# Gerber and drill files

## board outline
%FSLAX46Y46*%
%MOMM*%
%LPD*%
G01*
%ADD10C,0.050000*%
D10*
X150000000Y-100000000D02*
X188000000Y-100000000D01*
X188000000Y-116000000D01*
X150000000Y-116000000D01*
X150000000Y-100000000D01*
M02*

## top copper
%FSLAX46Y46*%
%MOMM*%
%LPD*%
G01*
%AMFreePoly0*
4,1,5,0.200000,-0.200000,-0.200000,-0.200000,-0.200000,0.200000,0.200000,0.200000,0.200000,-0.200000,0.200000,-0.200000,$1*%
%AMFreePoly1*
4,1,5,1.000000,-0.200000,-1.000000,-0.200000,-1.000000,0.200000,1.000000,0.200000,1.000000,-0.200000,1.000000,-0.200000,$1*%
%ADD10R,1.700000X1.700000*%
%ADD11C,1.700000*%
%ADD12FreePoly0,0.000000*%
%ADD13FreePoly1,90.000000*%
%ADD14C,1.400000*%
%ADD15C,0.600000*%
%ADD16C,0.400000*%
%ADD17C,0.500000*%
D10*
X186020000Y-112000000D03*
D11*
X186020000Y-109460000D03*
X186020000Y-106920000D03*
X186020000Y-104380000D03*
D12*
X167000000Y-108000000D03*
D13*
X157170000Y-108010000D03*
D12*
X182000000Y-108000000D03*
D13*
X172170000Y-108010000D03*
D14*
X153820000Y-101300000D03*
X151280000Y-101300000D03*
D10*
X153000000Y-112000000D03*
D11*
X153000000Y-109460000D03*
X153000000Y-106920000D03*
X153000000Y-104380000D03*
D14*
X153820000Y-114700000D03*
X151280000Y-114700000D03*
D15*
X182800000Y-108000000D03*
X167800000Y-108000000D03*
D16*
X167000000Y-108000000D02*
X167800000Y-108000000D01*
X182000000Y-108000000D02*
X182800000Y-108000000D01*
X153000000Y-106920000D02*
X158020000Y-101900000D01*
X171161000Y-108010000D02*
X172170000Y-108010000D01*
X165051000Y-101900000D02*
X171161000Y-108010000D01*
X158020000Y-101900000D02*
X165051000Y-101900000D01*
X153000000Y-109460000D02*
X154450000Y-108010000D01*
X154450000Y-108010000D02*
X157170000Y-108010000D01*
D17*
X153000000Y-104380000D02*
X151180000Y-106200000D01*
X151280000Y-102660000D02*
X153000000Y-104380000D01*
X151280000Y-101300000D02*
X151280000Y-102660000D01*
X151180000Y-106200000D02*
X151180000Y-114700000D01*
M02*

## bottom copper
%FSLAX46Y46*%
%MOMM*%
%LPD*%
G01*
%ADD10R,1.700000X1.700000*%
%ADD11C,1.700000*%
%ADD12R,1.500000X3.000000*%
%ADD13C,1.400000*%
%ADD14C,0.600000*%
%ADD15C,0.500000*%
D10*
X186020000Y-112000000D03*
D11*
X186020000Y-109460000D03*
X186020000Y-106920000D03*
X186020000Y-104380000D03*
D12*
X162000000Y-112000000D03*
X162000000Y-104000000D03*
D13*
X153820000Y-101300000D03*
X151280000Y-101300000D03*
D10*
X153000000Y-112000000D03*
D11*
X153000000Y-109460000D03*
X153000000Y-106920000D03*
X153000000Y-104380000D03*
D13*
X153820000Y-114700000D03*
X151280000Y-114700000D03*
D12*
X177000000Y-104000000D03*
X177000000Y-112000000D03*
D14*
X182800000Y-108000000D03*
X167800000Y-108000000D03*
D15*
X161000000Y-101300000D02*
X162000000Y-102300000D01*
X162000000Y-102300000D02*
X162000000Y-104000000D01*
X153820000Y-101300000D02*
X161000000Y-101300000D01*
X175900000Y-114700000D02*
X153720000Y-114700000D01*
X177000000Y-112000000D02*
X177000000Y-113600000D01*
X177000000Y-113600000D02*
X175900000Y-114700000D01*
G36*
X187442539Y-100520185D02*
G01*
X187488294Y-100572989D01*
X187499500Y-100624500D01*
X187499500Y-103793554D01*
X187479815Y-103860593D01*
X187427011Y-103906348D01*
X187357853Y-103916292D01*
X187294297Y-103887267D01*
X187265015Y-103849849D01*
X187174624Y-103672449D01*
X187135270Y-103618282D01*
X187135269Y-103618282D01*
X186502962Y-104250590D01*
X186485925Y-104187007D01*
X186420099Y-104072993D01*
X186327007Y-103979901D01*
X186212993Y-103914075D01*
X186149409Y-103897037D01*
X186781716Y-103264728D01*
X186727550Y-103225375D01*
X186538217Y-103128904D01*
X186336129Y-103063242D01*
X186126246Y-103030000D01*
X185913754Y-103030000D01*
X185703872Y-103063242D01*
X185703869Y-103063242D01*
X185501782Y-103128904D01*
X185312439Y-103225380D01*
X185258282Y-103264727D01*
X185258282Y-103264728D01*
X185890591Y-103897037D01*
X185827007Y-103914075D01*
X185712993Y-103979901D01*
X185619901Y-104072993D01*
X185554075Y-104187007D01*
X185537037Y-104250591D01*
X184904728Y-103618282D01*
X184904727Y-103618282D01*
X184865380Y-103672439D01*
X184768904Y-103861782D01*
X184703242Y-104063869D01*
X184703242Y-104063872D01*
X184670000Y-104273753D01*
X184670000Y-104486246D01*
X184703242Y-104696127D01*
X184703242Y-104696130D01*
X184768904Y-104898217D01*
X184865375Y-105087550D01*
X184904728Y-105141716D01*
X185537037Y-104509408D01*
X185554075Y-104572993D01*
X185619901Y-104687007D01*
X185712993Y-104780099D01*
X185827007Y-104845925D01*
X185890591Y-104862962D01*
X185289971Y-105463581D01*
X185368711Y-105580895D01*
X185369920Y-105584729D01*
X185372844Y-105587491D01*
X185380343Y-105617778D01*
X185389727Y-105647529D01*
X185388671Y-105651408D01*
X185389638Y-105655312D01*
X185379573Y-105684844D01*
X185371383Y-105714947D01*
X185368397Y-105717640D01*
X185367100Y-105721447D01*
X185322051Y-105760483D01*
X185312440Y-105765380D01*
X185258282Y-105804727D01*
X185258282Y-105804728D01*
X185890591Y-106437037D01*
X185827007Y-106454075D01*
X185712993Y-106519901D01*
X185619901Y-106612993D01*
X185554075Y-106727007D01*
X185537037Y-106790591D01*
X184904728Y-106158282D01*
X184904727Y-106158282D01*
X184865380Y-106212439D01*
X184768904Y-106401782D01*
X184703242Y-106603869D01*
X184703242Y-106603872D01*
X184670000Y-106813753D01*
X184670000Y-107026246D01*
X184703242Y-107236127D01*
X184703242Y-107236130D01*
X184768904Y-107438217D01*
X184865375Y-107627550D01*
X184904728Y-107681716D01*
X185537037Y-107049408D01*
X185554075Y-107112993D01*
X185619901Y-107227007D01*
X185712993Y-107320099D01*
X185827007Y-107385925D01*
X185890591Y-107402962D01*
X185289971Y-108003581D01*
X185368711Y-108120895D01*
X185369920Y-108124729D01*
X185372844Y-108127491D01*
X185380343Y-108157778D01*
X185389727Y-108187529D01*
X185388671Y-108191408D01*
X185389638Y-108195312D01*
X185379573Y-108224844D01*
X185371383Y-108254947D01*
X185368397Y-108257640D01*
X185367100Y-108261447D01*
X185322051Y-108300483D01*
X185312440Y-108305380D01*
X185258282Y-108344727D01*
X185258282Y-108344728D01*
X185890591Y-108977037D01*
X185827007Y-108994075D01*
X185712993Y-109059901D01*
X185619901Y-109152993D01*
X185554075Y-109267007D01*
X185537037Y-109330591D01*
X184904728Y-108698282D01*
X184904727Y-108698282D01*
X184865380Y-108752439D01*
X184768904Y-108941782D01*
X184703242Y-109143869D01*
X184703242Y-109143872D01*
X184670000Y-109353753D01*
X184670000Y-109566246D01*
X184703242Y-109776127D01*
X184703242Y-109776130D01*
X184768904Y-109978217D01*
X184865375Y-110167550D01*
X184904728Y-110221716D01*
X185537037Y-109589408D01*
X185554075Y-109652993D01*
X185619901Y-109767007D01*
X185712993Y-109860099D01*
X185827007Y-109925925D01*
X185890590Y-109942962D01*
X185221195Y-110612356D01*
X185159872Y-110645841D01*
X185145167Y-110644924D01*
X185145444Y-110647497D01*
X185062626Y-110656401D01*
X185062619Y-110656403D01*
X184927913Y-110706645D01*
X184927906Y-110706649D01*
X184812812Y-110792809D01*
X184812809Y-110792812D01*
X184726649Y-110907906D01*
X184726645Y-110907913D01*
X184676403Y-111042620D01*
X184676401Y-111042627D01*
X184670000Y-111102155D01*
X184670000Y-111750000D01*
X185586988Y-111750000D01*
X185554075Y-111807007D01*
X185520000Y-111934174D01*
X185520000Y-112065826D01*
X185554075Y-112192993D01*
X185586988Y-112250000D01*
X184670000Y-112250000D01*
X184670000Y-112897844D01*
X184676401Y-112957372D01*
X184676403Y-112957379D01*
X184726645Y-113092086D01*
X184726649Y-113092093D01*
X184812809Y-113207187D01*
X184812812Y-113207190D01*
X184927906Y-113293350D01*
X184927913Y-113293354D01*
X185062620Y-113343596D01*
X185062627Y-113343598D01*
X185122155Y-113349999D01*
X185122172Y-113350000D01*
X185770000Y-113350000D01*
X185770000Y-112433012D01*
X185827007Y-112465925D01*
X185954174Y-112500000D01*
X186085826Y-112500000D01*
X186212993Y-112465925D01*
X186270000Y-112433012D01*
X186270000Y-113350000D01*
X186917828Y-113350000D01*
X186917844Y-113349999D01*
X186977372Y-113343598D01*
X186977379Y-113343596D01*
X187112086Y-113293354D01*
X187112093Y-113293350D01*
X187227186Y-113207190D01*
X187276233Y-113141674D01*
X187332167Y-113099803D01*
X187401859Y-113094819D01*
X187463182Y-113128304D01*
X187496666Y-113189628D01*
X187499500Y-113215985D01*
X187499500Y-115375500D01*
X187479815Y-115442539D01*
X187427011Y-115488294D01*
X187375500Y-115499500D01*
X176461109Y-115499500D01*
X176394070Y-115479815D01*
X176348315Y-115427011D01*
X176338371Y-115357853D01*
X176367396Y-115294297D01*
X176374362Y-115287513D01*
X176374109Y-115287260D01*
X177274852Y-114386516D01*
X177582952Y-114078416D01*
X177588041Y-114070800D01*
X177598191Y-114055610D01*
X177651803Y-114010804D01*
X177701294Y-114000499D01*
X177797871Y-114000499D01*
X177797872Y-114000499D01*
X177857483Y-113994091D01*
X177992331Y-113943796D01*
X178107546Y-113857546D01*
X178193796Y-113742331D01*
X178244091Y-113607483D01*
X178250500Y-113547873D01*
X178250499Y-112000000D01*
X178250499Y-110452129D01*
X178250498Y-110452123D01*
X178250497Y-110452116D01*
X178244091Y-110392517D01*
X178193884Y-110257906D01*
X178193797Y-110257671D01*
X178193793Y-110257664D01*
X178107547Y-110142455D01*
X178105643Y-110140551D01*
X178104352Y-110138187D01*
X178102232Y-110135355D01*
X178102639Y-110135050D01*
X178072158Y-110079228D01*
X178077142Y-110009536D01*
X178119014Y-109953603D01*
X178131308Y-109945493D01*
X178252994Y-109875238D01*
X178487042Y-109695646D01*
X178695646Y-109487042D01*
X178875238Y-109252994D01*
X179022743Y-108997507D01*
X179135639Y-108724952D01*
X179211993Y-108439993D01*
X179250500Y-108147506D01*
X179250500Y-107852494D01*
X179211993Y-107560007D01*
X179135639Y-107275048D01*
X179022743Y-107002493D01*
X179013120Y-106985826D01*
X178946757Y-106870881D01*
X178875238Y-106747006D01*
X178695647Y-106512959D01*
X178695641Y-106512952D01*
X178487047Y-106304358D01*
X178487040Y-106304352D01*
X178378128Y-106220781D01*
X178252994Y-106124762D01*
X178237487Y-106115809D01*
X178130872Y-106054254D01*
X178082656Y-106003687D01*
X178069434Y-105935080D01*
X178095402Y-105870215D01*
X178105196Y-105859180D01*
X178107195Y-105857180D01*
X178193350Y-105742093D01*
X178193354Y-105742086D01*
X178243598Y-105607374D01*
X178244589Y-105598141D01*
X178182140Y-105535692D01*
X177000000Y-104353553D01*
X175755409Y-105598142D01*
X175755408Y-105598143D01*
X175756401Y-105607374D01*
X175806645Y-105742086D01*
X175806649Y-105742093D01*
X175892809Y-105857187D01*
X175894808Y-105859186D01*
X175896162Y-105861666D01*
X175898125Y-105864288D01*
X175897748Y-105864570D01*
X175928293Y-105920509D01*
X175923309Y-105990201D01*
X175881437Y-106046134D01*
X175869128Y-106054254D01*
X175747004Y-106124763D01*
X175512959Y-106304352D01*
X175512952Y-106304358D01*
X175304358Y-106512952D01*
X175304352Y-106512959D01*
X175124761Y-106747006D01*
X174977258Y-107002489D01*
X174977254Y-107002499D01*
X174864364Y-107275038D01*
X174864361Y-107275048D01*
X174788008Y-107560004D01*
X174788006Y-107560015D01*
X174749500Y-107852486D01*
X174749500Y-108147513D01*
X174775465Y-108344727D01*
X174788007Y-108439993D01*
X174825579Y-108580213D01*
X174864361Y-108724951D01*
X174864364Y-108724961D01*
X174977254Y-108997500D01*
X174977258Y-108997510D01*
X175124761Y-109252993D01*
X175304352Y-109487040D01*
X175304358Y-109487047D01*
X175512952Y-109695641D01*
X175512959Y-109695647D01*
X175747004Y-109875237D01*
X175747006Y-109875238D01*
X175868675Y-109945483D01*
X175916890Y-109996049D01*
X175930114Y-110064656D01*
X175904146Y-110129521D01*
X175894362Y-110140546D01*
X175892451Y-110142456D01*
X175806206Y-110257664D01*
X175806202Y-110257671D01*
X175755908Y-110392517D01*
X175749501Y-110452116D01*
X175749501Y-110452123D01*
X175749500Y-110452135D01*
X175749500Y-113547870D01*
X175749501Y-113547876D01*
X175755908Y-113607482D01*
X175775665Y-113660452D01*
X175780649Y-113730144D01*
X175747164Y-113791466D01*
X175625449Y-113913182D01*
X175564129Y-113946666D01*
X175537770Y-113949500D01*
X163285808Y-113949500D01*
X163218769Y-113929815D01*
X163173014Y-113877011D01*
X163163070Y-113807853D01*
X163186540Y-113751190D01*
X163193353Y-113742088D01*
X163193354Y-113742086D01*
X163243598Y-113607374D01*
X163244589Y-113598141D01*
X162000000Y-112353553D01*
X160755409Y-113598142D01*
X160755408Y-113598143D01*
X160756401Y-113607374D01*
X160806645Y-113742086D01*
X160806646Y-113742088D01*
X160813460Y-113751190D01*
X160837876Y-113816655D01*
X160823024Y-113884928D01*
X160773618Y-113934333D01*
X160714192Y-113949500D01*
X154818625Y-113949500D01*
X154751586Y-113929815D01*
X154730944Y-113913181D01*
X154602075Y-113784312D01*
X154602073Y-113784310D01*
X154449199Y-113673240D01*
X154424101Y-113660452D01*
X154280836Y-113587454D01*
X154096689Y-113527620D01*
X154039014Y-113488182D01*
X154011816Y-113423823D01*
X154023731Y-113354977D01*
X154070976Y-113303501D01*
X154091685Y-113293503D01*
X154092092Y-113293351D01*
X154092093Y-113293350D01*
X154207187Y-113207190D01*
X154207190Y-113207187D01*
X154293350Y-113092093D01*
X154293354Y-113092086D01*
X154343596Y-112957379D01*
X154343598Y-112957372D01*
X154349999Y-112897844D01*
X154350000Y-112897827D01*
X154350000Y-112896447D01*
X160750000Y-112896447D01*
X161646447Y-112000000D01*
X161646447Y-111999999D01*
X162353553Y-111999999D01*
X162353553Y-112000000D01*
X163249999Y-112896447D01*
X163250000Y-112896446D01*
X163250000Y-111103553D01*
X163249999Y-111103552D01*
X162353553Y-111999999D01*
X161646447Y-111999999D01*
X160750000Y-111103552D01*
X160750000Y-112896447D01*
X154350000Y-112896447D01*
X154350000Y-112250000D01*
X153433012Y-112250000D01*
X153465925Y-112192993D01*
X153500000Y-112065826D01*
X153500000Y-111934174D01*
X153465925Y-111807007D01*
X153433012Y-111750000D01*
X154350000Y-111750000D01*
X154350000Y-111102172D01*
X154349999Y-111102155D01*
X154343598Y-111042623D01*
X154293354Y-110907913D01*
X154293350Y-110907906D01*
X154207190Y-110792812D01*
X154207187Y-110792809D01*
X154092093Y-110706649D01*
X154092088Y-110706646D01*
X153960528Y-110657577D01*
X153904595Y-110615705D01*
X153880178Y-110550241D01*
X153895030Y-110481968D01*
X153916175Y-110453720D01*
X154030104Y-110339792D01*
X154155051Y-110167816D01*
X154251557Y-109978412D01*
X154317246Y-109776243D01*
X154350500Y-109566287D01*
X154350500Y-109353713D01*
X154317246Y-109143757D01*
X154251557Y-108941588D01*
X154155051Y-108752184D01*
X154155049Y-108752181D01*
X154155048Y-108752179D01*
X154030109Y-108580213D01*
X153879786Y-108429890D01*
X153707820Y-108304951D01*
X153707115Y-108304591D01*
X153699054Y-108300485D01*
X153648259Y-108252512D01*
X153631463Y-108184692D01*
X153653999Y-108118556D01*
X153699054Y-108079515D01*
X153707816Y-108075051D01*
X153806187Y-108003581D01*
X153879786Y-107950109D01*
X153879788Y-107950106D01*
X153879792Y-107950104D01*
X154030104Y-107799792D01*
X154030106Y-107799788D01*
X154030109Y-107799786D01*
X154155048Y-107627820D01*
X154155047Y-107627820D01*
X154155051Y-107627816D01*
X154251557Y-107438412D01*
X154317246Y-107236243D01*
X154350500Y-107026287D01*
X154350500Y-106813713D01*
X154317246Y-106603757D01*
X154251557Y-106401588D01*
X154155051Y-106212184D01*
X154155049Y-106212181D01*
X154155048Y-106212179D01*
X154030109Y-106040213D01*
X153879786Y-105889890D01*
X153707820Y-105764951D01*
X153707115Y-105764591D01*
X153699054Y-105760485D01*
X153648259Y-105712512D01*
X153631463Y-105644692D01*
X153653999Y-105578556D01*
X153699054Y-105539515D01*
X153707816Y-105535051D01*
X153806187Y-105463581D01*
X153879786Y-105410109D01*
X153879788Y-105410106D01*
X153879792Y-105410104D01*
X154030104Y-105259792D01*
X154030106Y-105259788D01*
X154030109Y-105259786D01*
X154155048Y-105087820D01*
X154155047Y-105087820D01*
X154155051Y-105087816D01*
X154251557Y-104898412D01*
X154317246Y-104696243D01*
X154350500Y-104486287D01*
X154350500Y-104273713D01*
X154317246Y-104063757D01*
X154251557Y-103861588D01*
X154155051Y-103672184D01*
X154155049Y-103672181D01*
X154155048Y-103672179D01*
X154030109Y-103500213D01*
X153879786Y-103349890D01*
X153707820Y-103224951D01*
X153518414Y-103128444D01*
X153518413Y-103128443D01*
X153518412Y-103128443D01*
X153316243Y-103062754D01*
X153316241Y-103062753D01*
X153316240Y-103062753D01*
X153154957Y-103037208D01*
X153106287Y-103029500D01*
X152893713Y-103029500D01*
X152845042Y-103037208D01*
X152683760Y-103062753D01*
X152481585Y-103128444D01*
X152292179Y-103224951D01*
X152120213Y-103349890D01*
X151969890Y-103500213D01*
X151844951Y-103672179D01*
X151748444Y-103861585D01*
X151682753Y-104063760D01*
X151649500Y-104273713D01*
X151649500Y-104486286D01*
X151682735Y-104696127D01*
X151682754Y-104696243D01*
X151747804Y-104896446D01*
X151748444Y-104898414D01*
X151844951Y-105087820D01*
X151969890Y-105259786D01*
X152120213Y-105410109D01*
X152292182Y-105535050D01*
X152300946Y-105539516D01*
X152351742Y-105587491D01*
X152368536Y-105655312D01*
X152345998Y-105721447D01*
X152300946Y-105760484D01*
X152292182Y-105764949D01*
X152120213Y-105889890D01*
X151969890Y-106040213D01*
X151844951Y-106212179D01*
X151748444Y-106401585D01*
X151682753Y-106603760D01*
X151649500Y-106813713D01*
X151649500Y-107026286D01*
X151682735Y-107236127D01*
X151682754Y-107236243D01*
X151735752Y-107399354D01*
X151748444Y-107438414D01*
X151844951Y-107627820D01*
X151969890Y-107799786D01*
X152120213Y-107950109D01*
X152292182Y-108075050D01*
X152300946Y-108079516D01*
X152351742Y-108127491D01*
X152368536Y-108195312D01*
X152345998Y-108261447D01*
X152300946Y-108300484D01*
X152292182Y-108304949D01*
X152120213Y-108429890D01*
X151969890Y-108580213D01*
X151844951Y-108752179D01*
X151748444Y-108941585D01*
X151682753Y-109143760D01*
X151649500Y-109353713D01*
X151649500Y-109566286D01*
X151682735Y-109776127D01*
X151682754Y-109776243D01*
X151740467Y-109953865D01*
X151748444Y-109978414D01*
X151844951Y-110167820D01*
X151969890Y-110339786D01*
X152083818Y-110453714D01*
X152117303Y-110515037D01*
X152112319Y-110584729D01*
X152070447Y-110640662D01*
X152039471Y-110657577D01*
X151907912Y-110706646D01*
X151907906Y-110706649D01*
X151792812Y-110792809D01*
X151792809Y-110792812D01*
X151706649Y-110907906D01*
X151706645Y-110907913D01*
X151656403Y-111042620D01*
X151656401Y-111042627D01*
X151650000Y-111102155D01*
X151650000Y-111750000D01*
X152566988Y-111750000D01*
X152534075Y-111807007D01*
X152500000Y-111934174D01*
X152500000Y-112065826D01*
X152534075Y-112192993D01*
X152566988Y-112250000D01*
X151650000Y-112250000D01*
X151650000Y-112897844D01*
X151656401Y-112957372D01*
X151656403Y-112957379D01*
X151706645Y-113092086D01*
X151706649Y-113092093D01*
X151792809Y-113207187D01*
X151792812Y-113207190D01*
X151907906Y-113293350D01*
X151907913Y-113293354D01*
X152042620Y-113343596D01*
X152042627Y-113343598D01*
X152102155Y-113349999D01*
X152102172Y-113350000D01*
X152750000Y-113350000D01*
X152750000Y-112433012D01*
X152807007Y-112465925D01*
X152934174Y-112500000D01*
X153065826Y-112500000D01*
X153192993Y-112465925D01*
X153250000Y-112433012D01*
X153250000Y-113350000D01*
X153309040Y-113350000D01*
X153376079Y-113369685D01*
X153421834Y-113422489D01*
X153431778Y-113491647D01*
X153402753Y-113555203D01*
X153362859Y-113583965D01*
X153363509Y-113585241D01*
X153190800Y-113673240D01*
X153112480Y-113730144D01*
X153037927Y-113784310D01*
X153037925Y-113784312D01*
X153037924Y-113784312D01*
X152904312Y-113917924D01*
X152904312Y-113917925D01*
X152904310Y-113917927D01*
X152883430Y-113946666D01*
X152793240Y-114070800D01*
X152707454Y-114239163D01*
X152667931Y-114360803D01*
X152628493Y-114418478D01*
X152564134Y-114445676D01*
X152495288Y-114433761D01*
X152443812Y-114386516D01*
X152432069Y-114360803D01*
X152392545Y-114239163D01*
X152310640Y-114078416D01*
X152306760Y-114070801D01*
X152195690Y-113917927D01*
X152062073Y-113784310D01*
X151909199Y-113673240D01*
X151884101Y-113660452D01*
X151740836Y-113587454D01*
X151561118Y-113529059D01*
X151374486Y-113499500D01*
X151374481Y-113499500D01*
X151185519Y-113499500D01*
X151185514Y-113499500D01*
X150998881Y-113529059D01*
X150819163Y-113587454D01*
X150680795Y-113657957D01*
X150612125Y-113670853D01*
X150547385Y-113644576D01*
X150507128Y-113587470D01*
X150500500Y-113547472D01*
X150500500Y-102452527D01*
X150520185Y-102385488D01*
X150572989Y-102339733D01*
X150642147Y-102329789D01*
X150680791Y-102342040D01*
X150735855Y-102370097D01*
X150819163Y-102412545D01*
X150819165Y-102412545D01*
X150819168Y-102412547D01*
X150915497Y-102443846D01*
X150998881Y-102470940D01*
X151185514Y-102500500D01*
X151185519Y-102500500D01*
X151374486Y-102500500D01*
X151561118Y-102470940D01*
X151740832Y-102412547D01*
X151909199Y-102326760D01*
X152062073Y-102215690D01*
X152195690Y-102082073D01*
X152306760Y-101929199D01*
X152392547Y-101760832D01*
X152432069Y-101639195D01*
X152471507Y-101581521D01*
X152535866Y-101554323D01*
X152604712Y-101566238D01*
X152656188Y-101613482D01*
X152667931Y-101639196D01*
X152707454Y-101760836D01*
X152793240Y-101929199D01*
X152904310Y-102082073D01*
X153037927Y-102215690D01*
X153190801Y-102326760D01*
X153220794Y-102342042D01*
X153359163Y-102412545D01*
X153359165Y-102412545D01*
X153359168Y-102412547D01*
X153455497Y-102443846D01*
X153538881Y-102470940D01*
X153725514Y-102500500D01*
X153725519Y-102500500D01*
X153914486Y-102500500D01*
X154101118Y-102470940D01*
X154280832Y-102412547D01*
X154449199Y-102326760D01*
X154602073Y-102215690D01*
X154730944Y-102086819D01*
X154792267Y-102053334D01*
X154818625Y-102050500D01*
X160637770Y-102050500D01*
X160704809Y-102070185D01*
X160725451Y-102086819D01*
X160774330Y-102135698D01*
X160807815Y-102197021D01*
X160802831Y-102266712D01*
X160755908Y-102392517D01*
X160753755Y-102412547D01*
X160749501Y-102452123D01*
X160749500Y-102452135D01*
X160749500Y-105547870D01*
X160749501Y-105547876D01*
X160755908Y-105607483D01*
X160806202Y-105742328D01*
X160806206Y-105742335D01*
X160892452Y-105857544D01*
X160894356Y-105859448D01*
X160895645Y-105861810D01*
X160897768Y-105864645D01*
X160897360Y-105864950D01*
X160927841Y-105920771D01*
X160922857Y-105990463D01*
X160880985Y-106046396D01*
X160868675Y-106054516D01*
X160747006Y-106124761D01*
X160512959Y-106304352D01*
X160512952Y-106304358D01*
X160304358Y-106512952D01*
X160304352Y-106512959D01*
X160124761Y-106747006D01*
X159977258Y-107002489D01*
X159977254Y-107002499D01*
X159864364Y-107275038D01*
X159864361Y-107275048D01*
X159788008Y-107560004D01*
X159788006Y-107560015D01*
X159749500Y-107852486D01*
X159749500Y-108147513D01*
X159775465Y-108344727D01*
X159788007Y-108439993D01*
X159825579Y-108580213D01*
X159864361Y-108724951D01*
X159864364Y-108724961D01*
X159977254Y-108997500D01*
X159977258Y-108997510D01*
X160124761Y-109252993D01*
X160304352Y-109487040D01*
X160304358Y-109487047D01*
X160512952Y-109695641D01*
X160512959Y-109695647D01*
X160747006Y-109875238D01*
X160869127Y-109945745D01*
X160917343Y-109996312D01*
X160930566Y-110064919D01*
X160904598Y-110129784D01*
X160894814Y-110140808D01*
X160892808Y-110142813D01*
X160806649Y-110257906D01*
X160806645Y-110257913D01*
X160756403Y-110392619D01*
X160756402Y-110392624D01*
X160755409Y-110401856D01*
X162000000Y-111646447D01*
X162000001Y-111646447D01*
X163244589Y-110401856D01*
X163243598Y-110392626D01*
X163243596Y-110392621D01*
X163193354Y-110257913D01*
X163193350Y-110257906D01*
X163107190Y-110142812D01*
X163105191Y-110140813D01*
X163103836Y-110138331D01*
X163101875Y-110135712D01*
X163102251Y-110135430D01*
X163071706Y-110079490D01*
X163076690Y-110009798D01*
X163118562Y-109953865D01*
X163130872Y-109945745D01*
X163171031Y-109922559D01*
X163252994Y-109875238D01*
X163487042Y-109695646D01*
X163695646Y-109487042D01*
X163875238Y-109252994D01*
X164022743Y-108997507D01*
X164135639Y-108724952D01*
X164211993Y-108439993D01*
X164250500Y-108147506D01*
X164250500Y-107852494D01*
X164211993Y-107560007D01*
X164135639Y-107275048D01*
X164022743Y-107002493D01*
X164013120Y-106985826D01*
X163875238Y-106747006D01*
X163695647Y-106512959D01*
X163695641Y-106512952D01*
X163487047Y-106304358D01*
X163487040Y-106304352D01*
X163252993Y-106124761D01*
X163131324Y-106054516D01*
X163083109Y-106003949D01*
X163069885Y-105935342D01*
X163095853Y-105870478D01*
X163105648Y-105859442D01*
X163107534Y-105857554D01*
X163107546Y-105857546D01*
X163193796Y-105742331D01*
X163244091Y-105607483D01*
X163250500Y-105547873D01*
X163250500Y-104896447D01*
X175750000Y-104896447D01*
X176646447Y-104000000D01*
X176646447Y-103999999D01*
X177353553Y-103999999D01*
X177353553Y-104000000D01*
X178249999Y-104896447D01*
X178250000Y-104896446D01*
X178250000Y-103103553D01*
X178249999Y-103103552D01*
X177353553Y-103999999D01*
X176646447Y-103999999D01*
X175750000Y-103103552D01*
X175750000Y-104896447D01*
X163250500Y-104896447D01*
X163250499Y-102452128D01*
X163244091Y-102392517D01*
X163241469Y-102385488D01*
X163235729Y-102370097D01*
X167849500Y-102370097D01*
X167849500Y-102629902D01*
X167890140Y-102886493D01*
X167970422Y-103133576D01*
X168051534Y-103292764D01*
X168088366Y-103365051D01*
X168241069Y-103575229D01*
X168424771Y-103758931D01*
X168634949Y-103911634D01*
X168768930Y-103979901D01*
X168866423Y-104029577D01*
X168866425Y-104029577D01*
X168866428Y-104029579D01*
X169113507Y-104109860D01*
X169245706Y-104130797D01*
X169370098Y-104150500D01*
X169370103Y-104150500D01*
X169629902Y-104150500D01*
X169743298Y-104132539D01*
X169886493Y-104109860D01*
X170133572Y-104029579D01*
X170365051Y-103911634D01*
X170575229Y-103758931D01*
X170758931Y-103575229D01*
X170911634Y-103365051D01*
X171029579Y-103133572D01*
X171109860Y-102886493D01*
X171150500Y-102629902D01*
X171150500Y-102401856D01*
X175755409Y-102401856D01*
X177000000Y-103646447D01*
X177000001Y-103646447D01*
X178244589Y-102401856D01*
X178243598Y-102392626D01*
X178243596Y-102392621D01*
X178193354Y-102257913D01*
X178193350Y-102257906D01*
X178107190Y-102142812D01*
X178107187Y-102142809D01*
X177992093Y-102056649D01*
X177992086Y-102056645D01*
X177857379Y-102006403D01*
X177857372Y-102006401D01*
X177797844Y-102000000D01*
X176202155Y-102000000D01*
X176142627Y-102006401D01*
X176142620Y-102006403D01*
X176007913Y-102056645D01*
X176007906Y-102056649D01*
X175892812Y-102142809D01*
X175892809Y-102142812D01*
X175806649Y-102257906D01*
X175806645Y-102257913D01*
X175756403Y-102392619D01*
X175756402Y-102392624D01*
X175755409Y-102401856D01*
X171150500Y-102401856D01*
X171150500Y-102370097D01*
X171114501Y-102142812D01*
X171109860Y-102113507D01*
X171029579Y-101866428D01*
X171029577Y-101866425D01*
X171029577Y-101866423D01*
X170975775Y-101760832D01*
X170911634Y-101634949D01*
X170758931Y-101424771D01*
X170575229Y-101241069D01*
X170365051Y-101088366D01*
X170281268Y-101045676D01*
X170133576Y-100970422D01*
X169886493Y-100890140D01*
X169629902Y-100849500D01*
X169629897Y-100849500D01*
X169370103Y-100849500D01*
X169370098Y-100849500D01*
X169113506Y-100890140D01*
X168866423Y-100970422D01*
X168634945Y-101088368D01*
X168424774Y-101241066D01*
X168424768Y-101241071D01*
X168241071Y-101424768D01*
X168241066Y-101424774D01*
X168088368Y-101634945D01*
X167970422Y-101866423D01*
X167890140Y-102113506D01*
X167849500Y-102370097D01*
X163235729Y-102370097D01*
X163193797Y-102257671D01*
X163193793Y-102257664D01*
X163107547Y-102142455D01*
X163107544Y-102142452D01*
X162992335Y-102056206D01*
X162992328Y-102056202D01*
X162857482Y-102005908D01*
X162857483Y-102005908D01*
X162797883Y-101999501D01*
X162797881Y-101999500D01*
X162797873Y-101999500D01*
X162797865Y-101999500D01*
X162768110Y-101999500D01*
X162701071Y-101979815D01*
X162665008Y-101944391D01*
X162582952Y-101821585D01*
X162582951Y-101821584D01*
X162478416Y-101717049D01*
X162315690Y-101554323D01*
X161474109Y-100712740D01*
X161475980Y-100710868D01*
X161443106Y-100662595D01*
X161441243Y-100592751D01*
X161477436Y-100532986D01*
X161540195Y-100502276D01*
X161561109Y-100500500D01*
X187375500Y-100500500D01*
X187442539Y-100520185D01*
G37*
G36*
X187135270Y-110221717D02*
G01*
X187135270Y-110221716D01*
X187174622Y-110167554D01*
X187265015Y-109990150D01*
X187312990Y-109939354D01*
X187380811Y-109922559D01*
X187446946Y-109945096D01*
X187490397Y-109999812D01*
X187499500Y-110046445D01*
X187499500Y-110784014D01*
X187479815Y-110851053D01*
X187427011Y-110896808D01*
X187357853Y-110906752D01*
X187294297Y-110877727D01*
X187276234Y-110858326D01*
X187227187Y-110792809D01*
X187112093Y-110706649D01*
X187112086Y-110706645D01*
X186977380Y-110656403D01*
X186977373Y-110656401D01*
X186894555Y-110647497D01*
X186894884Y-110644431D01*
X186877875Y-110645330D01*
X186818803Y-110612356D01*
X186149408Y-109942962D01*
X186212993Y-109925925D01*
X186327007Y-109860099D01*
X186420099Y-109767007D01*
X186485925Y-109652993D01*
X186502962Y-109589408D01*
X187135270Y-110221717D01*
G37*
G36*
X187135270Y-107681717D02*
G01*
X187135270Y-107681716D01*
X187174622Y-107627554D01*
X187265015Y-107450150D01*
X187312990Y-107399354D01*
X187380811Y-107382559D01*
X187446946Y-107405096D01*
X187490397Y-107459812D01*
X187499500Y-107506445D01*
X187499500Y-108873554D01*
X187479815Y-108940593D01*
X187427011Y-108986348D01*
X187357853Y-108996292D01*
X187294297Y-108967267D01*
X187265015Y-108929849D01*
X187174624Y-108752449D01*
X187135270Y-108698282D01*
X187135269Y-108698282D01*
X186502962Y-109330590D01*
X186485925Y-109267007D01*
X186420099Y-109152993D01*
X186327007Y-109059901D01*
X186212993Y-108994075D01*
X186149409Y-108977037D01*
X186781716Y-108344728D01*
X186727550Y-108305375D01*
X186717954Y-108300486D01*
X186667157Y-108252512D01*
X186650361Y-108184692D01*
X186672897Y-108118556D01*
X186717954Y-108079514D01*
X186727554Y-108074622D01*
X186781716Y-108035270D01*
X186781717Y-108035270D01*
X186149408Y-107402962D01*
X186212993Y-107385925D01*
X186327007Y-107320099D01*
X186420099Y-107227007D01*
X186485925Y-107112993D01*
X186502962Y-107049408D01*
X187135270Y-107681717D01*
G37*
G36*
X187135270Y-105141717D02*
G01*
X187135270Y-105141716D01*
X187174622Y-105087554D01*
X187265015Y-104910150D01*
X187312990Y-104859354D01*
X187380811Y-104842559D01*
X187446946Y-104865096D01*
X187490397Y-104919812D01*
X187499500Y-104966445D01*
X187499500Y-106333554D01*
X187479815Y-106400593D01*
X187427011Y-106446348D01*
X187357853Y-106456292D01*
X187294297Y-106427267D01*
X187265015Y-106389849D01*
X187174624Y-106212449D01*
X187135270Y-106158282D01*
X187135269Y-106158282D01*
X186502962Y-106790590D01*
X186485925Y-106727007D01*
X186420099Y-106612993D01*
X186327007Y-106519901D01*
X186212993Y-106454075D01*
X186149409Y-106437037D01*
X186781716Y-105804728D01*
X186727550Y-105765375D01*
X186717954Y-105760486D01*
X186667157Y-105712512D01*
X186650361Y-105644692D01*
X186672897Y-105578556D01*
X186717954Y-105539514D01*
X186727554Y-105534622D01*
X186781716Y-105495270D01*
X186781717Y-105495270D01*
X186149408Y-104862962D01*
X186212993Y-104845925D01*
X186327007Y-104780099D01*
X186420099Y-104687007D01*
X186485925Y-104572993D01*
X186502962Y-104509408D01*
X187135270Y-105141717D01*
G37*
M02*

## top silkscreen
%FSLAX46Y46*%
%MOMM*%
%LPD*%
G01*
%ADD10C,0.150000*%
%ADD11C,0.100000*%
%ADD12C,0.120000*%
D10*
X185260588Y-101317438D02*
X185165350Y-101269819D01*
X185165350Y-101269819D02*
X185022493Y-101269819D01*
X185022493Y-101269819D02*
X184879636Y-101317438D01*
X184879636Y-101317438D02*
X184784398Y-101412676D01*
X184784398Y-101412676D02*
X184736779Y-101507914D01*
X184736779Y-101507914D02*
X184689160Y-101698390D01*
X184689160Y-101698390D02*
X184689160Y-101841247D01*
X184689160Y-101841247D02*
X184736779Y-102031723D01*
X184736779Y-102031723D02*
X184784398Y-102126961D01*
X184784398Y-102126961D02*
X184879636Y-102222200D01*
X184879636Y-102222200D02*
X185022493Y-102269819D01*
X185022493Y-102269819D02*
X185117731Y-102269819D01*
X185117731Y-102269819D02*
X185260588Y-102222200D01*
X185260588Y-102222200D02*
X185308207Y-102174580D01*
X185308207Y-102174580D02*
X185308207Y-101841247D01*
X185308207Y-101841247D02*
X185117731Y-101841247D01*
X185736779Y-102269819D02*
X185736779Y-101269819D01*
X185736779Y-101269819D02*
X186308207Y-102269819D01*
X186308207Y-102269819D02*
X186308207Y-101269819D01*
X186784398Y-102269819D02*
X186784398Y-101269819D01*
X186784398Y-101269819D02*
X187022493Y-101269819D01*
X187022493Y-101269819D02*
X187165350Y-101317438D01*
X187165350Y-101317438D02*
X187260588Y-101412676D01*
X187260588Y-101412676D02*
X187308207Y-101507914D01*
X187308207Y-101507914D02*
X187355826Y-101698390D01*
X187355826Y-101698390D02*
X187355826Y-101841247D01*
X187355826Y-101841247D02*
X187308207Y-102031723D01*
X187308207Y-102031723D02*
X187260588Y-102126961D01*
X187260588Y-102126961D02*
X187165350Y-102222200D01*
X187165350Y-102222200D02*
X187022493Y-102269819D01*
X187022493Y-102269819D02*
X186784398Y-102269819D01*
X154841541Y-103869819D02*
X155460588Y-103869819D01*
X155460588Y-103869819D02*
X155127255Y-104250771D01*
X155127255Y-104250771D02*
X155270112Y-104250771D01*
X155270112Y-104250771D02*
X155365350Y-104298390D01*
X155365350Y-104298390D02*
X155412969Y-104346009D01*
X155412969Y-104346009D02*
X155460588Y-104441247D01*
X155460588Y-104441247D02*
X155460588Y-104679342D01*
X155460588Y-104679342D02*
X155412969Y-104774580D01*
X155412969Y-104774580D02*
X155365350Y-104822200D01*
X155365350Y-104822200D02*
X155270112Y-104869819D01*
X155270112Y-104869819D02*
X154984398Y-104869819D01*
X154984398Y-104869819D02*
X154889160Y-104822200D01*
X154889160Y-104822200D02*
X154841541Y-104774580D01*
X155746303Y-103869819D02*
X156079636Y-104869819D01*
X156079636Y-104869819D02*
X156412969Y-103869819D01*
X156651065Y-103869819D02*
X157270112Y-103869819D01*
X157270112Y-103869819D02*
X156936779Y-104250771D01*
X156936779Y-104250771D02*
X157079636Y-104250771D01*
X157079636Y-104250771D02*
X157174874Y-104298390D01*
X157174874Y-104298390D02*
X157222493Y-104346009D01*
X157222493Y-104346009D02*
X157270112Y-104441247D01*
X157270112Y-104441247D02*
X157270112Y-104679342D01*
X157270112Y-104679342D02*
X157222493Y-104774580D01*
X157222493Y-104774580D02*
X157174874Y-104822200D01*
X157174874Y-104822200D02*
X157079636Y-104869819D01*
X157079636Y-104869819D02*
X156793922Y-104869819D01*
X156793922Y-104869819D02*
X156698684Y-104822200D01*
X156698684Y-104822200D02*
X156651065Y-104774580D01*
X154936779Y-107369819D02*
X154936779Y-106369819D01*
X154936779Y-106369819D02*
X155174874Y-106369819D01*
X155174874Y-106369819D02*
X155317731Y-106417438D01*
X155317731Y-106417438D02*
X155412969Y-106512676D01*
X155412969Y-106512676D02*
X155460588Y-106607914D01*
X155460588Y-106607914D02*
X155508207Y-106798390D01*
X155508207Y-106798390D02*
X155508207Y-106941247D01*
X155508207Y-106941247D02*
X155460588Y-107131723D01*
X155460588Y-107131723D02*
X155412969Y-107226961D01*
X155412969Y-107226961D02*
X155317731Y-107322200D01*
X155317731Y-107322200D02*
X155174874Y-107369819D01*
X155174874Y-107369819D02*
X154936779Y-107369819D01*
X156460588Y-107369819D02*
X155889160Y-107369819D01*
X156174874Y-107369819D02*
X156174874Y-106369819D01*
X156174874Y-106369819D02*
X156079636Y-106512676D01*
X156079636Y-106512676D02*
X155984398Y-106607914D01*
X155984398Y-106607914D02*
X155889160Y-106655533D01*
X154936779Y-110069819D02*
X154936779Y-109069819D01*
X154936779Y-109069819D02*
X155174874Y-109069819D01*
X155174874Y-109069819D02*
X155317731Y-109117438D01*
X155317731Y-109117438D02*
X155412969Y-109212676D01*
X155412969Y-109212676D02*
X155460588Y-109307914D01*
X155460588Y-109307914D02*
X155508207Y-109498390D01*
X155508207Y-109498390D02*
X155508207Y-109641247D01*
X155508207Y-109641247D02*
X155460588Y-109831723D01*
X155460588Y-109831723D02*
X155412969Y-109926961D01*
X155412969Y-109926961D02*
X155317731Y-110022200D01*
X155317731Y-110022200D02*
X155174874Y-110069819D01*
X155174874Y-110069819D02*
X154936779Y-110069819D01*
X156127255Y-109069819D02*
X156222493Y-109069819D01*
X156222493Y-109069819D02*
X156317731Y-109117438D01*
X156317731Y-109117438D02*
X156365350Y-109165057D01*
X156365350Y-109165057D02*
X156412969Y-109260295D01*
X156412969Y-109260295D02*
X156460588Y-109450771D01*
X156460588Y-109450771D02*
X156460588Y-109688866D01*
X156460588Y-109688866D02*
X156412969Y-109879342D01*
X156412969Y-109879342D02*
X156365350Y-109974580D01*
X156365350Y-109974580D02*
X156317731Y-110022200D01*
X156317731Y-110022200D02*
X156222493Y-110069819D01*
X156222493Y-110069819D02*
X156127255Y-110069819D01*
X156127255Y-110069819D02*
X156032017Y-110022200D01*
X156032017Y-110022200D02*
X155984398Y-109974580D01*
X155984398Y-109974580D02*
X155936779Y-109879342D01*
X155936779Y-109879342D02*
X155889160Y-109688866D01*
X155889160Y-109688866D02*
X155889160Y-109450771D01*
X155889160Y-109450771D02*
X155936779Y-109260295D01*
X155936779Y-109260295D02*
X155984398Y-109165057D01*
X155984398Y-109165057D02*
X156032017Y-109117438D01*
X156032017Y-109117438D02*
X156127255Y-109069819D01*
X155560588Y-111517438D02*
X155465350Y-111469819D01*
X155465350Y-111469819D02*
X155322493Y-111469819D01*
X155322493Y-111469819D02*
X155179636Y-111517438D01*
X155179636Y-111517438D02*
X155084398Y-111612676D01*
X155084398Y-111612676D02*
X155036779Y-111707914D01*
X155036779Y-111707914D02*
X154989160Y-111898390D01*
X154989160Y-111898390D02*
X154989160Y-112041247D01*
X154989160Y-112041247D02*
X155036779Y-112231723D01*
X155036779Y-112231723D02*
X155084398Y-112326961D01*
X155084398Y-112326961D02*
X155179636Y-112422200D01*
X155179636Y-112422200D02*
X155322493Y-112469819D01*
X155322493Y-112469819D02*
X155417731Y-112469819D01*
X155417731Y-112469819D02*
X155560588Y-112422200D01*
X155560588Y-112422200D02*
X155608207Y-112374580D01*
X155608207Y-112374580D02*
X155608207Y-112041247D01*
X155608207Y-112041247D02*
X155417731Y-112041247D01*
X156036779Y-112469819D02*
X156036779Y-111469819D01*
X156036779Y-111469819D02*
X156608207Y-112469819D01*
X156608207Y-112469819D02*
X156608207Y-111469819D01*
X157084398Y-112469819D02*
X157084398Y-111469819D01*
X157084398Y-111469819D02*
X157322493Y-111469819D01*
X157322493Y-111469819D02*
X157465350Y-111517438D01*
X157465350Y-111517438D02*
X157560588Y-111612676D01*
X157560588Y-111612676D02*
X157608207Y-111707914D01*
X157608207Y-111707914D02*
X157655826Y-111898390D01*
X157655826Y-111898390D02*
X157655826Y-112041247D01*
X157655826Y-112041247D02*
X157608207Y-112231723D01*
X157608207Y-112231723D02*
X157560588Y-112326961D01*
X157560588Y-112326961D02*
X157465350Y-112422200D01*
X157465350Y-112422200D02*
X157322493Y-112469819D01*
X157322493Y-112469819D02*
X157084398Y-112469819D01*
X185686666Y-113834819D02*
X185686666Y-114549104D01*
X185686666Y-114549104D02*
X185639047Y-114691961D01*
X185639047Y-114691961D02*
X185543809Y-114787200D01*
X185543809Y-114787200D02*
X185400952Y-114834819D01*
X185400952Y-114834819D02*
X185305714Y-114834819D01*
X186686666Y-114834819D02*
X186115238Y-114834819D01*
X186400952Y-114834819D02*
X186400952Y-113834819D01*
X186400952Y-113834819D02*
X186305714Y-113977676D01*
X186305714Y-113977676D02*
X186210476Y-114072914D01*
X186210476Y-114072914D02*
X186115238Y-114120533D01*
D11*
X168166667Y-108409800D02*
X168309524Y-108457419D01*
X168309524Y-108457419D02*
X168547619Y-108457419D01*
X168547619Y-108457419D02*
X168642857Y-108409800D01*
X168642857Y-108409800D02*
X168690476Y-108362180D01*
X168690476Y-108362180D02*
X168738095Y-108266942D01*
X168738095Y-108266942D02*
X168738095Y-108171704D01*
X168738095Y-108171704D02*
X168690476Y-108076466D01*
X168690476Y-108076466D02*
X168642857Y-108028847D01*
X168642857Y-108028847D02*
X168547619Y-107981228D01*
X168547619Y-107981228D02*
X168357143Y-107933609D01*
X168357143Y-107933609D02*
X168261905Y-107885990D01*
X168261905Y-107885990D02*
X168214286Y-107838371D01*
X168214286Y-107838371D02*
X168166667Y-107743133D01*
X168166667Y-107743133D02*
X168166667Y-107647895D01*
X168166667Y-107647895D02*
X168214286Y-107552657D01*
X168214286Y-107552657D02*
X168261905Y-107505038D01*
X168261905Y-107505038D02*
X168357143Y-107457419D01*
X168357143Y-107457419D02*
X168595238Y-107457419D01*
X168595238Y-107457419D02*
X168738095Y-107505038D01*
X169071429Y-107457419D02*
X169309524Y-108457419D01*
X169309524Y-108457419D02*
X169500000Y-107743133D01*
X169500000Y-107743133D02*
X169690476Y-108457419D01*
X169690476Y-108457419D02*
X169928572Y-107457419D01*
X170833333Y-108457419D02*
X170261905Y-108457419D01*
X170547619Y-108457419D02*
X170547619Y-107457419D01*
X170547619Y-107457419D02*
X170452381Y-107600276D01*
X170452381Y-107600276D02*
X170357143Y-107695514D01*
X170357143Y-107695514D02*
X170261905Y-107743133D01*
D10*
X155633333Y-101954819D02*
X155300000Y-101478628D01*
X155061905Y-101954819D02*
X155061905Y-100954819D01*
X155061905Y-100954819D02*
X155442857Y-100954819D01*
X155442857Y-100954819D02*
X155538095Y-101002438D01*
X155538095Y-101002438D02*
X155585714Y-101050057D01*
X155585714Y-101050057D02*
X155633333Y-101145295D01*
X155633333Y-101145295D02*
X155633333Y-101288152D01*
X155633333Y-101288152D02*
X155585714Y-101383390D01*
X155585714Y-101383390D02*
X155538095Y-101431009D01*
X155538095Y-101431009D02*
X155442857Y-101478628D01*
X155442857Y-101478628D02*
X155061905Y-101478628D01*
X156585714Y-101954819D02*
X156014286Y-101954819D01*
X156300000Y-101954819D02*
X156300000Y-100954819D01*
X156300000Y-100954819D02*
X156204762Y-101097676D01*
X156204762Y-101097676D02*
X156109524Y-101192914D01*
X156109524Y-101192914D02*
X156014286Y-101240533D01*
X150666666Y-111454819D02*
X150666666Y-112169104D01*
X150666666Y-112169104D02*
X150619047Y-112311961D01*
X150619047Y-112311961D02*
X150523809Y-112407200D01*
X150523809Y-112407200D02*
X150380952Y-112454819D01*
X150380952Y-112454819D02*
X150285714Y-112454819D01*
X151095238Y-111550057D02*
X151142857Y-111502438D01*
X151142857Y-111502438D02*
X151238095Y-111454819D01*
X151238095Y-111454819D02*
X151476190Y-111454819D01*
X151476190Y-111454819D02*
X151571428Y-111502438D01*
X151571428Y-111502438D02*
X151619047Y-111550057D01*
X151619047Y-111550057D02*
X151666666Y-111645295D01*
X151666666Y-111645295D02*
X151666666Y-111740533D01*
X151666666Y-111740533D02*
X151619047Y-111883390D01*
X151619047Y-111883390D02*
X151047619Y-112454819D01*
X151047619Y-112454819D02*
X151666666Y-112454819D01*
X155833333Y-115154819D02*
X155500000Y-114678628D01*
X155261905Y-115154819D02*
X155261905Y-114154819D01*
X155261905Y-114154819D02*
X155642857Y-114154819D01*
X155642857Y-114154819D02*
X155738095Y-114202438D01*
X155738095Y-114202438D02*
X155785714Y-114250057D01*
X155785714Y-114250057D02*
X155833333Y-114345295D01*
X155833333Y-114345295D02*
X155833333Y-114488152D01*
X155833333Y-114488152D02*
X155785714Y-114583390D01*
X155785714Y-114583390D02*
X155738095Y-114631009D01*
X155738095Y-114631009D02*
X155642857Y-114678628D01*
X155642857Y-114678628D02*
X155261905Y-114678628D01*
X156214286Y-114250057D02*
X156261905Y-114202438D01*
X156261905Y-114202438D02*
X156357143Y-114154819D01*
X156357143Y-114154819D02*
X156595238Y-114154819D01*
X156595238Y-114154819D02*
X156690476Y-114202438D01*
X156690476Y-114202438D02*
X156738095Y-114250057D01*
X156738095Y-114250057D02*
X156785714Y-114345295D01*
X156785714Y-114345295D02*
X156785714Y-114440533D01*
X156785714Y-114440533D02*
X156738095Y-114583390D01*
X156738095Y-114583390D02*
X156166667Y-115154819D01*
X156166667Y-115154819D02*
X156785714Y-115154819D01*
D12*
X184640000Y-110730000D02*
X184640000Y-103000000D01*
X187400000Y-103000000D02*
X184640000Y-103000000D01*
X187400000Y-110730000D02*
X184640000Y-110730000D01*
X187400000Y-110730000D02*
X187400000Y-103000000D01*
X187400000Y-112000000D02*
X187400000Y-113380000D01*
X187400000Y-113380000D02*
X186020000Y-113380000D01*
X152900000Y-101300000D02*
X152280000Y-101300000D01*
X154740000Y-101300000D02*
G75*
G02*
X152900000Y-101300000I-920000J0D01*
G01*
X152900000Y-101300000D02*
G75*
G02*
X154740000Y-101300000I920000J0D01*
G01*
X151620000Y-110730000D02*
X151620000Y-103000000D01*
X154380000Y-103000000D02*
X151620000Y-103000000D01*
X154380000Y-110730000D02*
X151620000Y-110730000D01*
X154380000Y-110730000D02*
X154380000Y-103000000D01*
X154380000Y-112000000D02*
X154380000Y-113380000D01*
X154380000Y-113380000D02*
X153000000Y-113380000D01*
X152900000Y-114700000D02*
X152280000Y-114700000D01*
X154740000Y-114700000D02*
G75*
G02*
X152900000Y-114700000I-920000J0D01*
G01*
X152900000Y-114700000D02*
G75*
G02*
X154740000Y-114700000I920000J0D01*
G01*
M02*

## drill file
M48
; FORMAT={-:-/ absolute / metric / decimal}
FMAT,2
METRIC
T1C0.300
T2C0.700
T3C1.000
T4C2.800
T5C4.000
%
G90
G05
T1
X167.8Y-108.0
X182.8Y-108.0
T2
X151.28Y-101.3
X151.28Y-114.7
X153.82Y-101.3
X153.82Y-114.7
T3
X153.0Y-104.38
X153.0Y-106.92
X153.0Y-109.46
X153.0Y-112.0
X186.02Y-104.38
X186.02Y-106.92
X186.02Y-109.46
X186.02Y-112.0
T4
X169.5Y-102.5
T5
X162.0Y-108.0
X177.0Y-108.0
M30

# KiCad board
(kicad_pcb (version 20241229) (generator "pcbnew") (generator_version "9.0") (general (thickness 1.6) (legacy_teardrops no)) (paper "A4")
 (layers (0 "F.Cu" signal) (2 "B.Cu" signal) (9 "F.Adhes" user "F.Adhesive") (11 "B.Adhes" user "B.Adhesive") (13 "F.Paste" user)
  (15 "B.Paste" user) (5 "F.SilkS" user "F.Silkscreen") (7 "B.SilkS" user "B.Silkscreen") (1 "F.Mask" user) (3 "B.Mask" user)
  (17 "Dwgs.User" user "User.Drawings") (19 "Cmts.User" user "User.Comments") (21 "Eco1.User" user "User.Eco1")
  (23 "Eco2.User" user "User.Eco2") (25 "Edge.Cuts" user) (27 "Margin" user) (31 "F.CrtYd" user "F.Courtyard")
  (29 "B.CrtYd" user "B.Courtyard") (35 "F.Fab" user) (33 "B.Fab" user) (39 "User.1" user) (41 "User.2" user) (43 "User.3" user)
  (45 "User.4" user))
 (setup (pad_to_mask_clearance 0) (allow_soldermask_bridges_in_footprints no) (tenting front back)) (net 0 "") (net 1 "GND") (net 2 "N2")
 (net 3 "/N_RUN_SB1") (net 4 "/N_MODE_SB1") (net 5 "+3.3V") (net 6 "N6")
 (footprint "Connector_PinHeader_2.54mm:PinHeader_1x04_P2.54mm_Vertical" (layer "F.Cu") (at 186.02 112 180)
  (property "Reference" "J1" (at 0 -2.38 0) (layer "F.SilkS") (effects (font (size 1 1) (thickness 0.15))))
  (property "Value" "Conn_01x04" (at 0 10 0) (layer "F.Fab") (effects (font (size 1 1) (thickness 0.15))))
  (fp_line (start 1.38 1.27) (end 1.38 9) (stroke (width 0.12) (type solid)) (layer "F.SilkS"))
  (fp_line (start -1.38 9) (end 1.38 9) (stroke (width 0.12) (type solid)) (layer "F.SilkS"))
  (fp_line (start -1.38 1.27) (end 1.38 1.27) (stroke (width 0.12) (type solid)) (layer "F.SilkS"))
  (fp_line (start -1.38 1.27) (end -1.38 9) (stroke (width 0.12) (type solid)) (layer "F.SilkS"))
  (fp_line (start -1.38 0) (end -1.38 -1.38) (stroke (width 0.12) (type solid)) (layer "F.SilkS"))
  (fp_line (start -1.38 -1.38) (end 0 -1.38) (stroke (width 0.12) (type solid)) (layer "F.SilkS"))
  (pad "1" thru_hole rect (at 0 0 180) (size 1.7 1.7) (drill 1) (layers "*.Cu" "*.Mask") (remove_unused_layers no) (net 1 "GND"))
  (pad "2" thru_hole circle (at 0 2.54 180) (size 1.7 1.7) (drill 1) (layers "*.Cu" "*.Mask") (remove_unused_layers no) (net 1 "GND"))
  (pad "3" thru_hole circle (at 0 5.08 180) (size 1.7 1.7) (drill 1) (layers "*.Cu" "*.Mask") (remove_unused_layers no) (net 1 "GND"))
  (pad "4" thru_hole circle (at 0 7.62 180) (size 1.7 1.7) (drill 1) (layers "*.Cu" "*.Mask") (remove_unused_layers no) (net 1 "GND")))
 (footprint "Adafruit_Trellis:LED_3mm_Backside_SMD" (layer "F.Cu") (at 162 108 90)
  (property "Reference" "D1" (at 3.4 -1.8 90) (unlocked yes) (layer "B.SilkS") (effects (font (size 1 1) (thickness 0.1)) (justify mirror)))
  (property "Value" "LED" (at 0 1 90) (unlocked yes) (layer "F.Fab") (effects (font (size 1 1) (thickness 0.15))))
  (pad "" np_thru_hole circle (at 0 0 90) (size 4 4) (drill 4) (layers "*.Cu" "*.Mask"))
  (pad "1" smd rect (at -4 0 90) (size 3 1.5) (layers "B.Cu" "B.Mask" "B.Paste") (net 1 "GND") (thermal_bridge_angle 45))
  (pad "2" smd rect (at 4 0 90) (size 3 1.5) (layers "B.Cu" "B.Mask" "B.Paste") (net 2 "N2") (thermal_bridge_angle 45)))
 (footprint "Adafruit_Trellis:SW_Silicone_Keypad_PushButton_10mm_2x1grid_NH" (layer "F.Cu") (at 169.5 108)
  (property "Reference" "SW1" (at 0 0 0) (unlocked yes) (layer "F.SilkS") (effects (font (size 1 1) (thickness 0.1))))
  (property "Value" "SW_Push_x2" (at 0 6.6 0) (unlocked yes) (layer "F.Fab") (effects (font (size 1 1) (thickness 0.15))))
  (pad "" np_thru_hole circle (at 0 -5.5 90) (size 2.8 2.8) (drill 2.8) (layers "*.Cu" "*.Mask"))
  (pad "1" smd custom (at -2.5 0) (size 0.4 0.4) (layers "F.Cu" "F.Mask") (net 1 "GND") (solder_mask_margin 0.1016) (thermal_bridge_angle 0)
   (options (clearance outline) (anchor rect)) (primitives))
  (pad "2" smd custom (at -12.33 0.01 90) (size 2 0.4) (layers "F.Cu" "F.Mask") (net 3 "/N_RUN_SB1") (solder_mask_margin 0.1016)
   (thermal_bridge_angle 0) (options (clearance outline) (anchor rect)) (primitives))
  (pad "3" smd custom (at 12.5 0) (size 0.4 0.4) (layers "F.Cu" "F.Mask") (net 1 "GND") (solder_mask_margin 0.1016) (thermal_bridge_angle 0)
   (options (clearance outline) (anchor rect)) (primitives))
  (pad "4" smd custom (at 2.67 0.01 90) (size 2 0.4) (layers "F.Cu" "F.Mask") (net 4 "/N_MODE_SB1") (solder_mask_margin 0.1016)
   (thermal_bridge_angle 0) (options (clearance outline) (anchor rect)) (primitives)))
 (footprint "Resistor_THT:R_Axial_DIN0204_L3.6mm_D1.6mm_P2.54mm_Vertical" (layer "F.Cu") (at 153.82 101.3 180)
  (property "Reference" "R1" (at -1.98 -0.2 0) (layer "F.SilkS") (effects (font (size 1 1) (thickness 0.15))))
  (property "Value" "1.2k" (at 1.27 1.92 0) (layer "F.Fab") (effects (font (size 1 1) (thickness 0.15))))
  (fp_line (start 0.92 0) (end 1.54 0) (stroke (width 0.12) (type solid)) (layer "F.SilkS"))
  (fp_circle (center 0 0) (end 0.92 0) (stroke (width 0.12) (type solid)) (fill no) (layer "F.SilkS"))
  (pad "1" thru_hole circle (at 0 0 180) (size 1.4 1.4) (drill 0.7) (layers "*.Cu" "*.Mask") (remove_unused_layers no) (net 2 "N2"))
  (pad "2" thru_hole circle (at 2.54 0 180) (size 1.4 1.4) (drill 0.7) (layers "*.Cu" "*.Mask") (remove_unused_layers no) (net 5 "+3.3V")))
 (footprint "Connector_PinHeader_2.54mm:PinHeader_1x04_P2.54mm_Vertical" (layer "F.Cu") (at 153 112 180)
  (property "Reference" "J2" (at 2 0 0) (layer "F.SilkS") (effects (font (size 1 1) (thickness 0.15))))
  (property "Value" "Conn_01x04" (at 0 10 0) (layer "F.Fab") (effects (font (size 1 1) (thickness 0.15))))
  (fp_line (start 1.38 1.27) (end 1.38 9) (stroke (width 0.12) (type solid)) (layer "F.SilkS"))
  (fp_line (start -1.38 9) (end 1.38 9) (stroke (width 0.12) (type solid)) (layer "F.SilkS"))
  (fp_line (start -1.38 1.27) (end 1.38 1.27) (stroke (width 0.12) (type solid)) (layer "F.SilkS"))
  (fp_line (start -1.38 1.27) (end -1.38 9) (stroke (width 0.12) (type solid)) (layer "F.SilkS"))
  (fp_line (start -1.38 0) (end -1.38 -1.38) (stroke (width 0.12) (type solid)) (layer "F.SilkS"))
  (fp_line (start -1.38 -1.38) (end 0 -1.38) (stroke (width 0.12) (type solid)) (layer "F.SilkS"))
  (pad "1" thru_hole rect (at 0 0 180) (size 1.7 1.7) (drill 1) (layers "*.Cu" "*.Mask") (remove_unused_layers no) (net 1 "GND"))
  (pad "2" thru_hole circle (at 0 2.54 180) (size 1.7 1.7) (drill 1) (layers "*.Cu" "*.Mask") (remove_unused_layers no) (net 3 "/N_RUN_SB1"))
  (pad "3" thru_hole circle (at 0 5.08 180) (size 1.7 1.7) (drill 1) (layers "*.Cu" "*.Mask") (remove_unused_layers no)
   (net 4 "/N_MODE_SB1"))
  (pad "4" thru_hole circle (at 0 7.62 180) (size 1.7 1.7) (drill 1) (layers "*.Cu" "*.Mask") (remove_unused_layers no) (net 5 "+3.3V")))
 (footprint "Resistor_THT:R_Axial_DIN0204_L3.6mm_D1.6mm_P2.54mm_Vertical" (layer "F.Cu") (at 153.82 114.7 180)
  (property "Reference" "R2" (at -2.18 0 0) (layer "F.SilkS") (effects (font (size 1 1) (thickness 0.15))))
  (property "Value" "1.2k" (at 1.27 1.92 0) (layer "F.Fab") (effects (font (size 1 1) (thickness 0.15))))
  (fp_line (start 0.92 0) (end 1.54 0) (stroke (width 0.12) (type solid)) (layer "F.SilkS"))
  (fp_circle (center 0 0) (end 0.92 0) (stroke (width 0.12) (type solid)) (fill no) (layer "F.SilkS"))
  (pad "1" thru_hole circle (at 0 0 180) (size 1.4 1.4) (drill 0.7) (layers "*.Cu" "*.Mask") (remove_unused_layers no) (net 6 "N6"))
  (pad "2" thru_hole circle (at 2.54 0 180) (size 1.4 1.4) (drill 0.7) (layers "*.Cu" "*.Mask") (remove_unused_layers no) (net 5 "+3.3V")))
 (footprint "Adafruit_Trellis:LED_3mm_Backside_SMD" (layer "F.Cu") (at 177 108 -90)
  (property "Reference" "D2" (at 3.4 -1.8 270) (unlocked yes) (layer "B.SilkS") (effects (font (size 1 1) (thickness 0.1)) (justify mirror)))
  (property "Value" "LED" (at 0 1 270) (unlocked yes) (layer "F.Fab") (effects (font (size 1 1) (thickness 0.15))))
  (pad "" np_thru_hole circle (at 0 0 270) (size 4 4) (drill 4) (layers "*.Cu" "*.Mask"))
  (pad "1" smd rect (at -4 0 270) (size 3 1.5) (layers "B.Cu" "B.Mask" "B.Paste") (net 1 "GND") (thermal_bridge_angle 45))
  (pad "2" smd rect (at 4 0 270) (size 3 1.5) (layers "B.Cu" "B.Mask" "B.Paste") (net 6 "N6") (thermal_bridge_angle 45)))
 (gr_rect (start 150 100) (end 188 116) (stroke (width 0.05) (type default)) (fill no) (layer "Edge.Cuts"))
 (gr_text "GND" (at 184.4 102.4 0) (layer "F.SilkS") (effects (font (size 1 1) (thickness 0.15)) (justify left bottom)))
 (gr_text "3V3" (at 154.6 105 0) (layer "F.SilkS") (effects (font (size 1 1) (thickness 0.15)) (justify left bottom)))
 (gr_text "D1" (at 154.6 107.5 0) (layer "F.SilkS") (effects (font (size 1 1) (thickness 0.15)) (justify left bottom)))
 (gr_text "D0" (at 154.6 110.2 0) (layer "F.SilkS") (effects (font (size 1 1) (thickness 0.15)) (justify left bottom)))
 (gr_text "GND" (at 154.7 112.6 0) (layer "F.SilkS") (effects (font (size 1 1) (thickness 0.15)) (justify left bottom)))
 (segment (start 161 101.3) (end 162 102.3) (width 0.5) (layer "B.Cu") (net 2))
 (segment (start 162 102.3) (end 162 104) (width 0.5) (layer "B.Cu") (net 2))
 (segment (start 153.82 101.3) (end 161 101.3) (width 0.5) (layer "B.Cu") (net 2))
 (segment (start 167 108) (end 167.8 108) (width 0.4) (layer "F.Cu") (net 1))
 (segment (start 182 108) (end 182.8 108) (width 0.4) (layer "F.Cu") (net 1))
 (via (at 182.8 108) (size 0.6) (drill 0.3) (layers "F.Cu" "B.Cu") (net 1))
 (via (at 167.8 108) (size 0.6) (drill 0.3) (layers "F.Cu" "B.Cu") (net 1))
 (segment (start 175.9 114.7) (end 153.72 114.7) (width 0.5) (layer "B.Cu") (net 6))
 (segment (start 177 112) (end 177 113.6) (width 0.5) (layer "B.Cu") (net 6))
 (segment (start 177 113.6) (end 175.9 114.7) (width 0.5) (layer "B.Cu") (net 6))
 (segment (start 153 106.92) (end 158.02 101.9) (width 0.4) (layer "F.Cu") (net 4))
 (segment (start 171.161 108.01) (end 172.17 108.01) (width 0.4) (layer "F.Cu") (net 4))
 (segment (start 165.051 101.9) (end 171.161 108.01) (width 0.4) (layer "F.Cu") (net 4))
 (segment (start 158.02 101.9) (end 165.051 101.9) (width 0.4) (layer "F.Cu") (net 4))
 (segment (start 153 109.46) (end 154.45 108.01) (width 0.4) (layer "F.Cu") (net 3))
 (segment (start 154.45 108.01) (end 157.17 108.01) (width 0.4) (layer "F.Cu") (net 3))
 (segment (start 153 104.38) (end 151.18 106.2) (width 0.5) (layer "F.Cu") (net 5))
 (segment (start 151.28 102.66) (end 153 104.38) (width 0.5) (layer "F.Cu") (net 5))
 (segment (start 151.28 101.3) (end 151.28 102.66) (width 0.5) (layer "F.Cu") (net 5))
 (segment (start 151.18 106.2) (end 151.18 114.7) (width 0.5) (layer "F.Cu") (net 5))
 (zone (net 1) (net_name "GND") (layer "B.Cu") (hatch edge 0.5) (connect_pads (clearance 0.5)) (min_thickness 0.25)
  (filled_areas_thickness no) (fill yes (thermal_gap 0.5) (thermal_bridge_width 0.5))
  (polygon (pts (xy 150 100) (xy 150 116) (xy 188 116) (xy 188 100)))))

